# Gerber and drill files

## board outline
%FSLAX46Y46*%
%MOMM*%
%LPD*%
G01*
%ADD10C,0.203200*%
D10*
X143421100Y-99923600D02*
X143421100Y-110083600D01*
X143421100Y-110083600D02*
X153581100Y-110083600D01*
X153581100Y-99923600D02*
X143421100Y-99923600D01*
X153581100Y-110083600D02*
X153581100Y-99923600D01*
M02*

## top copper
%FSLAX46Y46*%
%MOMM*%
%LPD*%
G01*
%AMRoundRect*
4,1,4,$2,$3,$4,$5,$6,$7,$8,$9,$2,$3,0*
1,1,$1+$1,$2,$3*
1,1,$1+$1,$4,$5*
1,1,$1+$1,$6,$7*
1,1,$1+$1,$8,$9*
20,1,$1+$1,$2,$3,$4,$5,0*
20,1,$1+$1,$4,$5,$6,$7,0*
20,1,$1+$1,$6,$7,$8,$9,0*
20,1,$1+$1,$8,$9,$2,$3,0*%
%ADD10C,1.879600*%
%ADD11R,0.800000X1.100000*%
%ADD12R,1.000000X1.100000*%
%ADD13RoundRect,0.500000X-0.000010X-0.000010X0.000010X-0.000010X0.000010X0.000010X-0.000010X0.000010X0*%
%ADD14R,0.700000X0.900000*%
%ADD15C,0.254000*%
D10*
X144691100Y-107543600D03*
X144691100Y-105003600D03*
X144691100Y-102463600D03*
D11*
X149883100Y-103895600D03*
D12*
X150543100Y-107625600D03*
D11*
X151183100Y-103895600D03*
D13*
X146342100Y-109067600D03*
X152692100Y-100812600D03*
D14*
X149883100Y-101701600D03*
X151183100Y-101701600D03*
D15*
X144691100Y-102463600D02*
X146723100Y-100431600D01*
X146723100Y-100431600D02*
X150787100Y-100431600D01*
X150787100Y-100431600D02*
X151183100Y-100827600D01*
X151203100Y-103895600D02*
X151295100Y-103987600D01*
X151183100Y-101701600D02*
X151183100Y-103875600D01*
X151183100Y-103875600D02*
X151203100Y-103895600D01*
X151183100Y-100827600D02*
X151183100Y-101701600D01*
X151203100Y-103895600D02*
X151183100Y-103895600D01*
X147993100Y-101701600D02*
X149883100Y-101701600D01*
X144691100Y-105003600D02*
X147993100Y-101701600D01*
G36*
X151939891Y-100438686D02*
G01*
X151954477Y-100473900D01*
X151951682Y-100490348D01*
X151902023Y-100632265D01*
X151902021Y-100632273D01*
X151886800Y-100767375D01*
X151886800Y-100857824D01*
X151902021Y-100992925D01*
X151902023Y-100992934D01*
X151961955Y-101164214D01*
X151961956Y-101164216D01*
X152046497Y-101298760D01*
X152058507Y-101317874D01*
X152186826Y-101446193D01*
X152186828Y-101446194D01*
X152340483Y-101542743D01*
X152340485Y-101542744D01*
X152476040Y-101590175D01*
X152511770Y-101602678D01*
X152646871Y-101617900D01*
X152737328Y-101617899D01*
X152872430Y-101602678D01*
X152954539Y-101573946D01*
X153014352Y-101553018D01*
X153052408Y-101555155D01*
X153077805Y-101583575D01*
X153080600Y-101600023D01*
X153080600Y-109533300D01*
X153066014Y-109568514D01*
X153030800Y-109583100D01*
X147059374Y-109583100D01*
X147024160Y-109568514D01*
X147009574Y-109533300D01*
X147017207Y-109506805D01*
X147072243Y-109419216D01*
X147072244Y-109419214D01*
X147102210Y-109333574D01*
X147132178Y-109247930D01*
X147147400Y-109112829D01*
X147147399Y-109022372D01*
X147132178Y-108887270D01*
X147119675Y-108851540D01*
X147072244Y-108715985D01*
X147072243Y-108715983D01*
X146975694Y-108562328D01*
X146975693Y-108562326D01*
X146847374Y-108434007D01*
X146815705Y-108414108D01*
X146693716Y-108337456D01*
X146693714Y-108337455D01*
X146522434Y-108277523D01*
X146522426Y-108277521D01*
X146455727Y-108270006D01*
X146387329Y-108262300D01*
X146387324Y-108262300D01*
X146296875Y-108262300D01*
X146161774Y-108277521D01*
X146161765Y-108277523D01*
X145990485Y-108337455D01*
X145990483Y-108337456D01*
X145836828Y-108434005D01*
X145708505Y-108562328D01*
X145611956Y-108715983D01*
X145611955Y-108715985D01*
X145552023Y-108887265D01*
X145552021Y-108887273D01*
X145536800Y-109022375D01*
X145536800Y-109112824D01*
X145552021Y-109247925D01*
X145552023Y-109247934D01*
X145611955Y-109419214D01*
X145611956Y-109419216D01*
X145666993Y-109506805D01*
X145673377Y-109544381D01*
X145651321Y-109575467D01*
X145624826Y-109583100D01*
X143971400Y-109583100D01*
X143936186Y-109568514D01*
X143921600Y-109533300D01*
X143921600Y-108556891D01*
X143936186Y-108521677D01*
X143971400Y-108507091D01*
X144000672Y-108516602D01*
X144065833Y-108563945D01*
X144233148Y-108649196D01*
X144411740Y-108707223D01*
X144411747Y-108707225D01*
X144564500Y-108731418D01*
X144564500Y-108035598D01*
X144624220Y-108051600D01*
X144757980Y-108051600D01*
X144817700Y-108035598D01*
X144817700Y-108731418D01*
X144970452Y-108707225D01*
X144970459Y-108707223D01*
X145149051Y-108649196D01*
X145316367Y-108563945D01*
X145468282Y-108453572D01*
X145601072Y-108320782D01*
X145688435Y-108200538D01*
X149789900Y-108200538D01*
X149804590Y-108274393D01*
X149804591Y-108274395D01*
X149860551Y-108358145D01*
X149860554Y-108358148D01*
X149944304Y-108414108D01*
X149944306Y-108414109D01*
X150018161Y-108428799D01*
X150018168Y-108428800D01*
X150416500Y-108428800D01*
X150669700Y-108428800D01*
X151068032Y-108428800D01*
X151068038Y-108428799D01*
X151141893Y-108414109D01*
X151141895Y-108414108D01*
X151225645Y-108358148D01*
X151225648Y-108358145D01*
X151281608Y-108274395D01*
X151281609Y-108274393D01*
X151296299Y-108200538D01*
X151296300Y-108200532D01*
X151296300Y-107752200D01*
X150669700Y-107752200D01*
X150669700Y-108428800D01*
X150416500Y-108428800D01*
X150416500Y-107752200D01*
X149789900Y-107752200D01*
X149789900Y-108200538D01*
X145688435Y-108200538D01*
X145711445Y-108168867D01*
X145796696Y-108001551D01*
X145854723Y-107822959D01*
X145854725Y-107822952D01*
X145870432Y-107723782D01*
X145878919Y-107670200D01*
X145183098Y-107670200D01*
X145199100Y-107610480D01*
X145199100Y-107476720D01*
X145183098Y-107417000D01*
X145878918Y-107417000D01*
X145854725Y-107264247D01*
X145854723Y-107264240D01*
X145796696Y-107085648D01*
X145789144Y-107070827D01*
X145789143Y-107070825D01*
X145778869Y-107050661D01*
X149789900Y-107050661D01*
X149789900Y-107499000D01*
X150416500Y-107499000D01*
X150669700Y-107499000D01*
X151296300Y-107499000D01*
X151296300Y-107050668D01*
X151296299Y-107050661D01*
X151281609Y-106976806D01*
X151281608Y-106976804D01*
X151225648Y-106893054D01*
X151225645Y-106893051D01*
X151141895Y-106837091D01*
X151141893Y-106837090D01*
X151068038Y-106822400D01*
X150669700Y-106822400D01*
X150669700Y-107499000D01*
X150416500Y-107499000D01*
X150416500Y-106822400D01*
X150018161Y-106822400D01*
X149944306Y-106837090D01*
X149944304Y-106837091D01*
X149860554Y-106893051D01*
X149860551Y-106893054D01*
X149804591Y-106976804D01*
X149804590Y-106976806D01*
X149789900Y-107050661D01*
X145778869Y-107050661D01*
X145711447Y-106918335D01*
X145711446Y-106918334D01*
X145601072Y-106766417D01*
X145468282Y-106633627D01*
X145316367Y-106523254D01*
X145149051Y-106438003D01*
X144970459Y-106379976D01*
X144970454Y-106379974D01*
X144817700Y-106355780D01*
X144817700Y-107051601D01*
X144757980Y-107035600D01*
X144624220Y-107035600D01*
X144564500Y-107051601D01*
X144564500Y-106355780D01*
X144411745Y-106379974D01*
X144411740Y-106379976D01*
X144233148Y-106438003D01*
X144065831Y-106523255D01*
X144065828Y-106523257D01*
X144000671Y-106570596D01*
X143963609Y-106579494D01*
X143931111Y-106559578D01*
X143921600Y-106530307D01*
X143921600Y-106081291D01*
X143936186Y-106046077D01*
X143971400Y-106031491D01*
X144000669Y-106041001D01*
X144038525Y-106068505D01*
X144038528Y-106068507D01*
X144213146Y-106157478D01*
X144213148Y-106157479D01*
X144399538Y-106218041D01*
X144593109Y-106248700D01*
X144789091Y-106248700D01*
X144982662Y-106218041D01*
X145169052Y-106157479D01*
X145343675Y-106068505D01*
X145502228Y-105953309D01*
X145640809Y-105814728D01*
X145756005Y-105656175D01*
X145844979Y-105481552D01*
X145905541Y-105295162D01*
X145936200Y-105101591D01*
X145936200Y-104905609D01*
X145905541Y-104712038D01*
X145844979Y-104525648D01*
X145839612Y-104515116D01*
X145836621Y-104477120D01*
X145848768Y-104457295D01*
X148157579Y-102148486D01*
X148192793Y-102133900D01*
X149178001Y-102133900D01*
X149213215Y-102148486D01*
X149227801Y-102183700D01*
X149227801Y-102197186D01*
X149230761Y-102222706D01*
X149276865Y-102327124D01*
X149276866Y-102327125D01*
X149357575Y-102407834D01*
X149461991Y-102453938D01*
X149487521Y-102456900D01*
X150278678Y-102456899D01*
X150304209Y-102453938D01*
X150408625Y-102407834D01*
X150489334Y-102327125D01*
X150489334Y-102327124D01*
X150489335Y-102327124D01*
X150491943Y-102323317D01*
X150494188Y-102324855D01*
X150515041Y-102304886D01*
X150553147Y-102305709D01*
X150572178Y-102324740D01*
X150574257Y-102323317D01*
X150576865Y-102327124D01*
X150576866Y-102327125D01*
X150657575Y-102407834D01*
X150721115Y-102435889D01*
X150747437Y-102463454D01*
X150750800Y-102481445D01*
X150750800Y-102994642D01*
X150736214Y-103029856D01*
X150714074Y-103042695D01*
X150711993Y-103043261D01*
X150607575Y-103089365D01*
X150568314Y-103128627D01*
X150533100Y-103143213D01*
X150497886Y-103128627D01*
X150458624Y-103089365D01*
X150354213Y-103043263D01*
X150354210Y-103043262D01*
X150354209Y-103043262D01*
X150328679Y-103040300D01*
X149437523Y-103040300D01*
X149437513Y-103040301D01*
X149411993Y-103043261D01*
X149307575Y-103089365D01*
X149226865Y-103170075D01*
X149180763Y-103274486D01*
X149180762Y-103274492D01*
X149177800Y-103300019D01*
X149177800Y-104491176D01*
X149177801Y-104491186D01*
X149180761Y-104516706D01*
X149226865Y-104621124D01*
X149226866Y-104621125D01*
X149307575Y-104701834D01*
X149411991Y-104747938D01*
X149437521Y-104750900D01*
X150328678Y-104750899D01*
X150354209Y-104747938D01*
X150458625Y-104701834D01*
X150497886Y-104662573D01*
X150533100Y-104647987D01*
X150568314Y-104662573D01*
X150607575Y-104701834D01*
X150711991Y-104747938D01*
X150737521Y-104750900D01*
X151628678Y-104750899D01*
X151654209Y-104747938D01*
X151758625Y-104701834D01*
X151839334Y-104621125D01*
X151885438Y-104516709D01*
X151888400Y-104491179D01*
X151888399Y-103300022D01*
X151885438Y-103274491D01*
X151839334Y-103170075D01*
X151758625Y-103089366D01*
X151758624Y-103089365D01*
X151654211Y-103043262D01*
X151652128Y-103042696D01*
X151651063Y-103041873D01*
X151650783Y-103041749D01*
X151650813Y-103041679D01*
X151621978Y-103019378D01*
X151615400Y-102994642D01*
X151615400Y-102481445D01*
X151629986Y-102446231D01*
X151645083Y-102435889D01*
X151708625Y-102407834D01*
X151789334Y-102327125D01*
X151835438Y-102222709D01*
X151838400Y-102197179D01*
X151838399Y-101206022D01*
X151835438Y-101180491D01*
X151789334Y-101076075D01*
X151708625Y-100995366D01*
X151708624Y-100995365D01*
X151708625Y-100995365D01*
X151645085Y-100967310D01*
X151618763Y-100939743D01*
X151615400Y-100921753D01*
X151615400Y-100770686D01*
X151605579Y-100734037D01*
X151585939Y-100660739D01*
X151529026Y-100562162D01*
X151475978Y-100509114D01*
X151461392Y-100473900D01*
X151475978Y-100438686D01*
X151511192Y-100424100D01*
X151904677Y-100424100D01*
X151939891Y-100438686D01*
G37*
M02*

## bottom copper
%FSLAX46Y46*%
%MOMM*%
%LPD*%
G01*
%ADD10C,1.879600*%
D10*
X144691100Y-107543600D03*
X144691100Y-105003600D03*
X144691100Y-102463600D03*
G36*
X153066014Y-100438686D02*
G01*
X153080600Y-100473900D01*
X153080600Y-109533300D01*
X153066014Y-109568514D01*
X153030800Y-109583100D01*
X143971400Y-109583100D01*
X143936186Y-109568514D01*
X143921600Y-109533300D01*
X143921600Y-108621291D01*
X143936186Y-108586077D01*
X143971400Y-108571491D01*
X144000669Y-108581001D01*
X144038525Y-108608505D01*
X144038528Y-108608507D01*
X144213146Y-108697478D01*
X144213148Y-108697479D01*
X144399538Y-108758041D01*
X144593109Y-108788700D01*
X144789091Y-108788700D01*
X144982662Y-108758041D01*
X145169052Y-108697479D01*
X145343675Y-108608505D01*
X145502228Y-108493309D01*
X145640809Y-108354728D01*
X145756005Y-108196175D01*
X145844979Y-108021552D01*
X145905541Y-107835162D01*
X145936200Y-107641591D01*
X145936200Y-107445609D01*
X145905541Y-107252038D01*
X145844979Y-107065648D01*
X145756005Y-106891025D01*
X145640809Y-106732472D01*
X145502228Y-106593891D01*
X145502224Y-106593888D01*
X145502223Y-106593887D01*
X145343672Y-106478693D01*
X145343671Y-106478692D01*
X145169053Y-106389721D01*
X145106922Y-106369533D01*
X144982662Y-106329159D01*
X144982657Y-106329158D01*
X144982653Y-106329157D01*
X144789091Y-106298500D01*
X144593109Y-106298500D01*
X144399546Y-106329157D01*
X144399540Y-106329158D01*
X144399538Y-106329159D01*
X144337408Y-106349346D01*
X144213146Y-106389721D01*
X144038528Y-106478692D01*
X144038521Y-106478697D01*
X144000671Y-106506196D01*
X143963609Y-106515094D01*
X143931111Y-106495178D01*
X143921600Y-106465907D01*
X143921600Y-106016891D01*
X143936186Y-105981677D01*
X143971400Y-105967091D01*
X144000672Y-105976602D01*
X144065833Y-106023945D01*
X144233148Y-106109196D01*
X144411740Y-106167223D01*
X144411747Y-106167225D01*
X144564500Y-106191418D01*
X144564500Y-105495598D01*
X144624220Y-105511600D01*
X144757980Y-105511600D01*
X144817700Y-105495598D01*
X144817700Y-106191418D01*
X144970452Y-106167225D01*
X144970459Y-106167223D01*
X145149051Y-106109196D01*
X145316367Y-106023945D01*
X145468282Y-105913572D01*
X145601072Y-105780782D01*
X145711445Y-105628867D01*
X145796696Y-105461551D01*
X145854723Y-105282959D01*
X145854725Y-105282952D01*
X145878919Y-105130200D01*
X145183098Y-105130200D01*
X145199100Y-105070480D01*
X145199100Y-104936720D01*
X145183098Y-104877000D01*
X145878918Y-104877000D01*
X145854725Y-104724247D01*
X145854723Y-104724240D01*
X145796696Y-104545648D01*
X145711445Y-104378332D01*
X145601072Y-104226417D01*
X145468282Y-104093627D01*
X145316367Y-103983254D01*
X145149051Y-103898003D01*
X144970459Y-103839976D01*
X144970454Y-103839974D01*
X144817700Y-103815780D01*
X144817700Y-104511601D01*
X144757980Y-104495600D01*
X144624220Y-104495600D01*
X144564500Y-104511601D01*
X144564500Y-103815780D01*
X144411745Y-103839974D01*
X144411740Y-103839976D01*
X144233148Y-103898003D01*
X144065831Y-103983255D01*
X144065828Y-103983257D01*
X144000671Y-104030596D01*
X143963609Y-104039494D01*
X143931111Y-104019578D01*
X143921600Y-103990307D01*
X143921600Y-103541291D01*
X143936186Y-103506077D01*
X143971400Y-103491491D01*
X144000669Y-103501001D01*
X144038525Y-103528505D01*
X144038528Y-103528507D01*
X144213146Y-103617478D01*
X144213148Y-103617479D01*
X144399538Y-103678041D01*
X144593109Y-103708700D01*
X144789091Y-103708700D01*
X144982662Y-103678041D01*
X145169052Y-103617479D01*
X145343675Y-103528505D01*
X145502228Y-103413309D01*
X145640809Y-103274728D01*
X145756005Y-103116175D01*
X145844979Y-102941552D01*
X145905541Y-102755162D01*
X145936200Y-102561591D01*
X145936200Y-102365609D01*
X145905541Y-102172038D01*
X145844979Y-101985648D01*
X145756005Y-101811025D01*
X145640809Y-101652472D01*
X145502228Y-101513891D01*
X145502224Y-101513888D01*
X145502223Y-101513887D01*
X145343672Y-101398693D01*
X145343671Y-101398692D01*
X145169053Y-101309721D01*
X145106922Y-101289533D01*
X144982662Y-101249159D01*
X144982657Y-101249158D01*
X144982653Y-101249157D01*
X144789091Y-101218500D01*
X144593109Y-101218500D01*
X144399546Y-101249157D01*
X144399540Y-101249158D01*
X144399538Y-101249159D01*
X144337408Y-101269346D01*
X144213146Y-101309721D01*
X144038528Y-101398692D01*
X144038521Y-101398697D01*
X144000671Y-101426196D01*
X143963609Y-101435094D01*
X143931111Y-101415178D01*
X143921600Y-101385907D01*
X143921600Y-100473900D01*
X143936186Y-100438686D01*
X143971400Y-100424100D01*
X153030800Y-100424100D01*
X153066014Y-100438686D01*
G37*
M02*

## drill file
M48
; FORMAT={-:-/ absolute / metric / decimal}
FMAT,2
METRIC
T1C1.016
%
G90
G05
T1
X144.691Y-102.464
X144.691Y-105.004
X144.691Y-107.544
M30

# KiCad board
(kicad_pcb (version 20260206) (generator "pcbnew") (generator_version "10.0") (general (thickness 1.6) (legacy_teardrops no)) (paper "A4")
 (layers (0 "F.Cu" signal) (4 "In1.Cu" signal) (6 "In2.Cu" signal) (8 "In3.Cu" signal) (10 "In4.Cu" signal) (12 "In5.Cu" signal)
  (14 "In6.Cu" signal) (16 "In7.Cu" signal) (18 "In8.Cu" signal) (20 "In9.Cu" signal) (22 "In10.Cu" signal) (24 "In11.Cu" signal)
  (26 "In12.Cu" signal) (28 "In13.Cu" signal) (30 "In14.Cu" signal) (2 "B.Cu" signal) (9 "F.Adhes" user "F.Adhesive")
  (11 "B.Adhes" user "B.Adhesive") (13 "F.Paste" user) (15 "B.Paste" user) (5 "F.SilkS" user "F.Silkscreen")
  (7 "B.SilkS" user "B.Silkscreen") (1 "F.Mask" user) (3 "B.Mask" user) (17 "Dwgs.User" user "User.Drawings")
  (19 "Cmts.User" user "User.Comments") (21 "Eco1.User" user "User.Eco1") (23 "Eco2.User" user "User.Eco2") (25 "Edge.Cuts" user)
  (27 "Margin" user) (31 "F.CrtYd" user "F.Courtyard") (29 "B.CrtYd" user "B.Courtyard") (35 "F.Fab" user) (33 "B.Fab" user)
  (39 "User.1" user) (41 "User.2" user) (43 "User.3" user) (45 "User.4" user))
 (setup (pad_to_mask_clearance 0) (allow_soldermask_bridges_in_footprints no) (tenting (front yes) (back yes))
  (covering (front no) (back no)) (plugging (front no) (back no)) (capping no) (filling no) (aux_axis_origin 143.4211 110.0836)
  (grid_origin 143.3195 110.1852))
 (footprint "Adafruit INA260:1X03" (layer "F.Cu") (at 144.6911 107.5436 90)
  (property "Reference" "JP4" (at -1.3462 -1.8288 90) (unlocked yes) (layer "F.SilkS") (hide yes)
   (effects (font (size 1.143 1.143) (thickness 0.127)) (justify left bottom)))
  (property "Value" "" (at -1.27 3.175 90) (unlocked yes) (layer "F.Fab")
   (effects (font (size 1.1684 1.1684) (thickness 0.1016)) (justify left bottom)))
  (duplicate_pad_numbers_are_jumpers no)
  (pad "1" thru_hole circle (at 0 0 180) (size 1.8796 1.8796) (drill 1.016) (layers "*.Cu" "*.Mask") (remove_unused_layers no) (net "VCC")
   (solder_mask_margin 0.1016) (thermal_bridge_angle 0))
  (pad "2" thru_hole circle (at 2.54 0 180) (size 1.8796 1.8796) (drill 1.016) (layers "*.Cu" "*.Mask") (remove_unused_layers no)
   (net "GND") (solder_mask_margin 0.1016) (thermal_bridge_angle 0))
  (pad "3" thru_hole circle (at 5.08 0 180) (size 1.8796 1.8796) (drill 1.016) (layers "*.Cu" "*.Mask") (remove_unused_layers no) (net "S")
   (solder_mask_margin 0.1016) (thermal_bridge_angle 0)))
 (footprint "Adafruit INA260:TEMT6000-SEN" (layer "F.Cu") (at 150.5331 105.7656 -90)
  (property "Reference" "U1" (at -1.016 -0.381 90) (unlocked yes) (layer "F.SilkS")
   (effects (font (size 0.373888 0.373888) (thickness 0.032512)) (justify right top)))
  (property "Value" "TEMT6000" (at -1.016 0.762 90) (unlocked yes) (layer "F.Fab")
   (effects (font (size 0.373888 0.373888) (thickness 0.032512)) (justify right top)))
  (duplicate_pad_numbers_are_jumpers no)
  (pad "BASE" smd rect (at -1.87 0.65 270) (size 1.1 0.8) (layers "F.Cu" "F.Mask" "F.Paste") (solder_mask_margin 0.1016)
   (solder_paste_margin 0) (thermal_bridge_angle 0))
  (pad "COLLECTOR" smd rect (at 1.86 -0.01 270) (size 1.1 1) (layers "F.Cu" "F.Mask" "F.Paste") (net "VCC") (solder_mask_margin 0.1016)
   (solder_paste_margin 0) (thermal_bridge_angle 0))
  (pad "EMITTER" smd rect (at -1.87 -0.65 270) (size 1.1 0.8) (layers "F.Cu" "F.Mask" "F.Paste") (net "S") (solder_mask_margin 0.1016)
   (solder_paste_margin 0) (thermal_bridge_angle 0)))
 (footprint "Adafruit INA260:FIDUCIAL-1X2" (layer "F.Cu") (at 146.3421 109.0676)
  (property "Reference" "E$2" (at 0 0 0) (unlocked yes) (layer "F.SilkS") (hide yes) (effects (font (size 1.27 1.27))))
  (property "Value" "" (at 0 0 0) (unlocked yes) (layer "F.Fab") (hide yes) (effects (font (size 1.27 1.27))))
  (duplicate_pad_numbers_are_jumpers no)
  (pad "1" smd roundrect (at 0 0) (size 1 1) (layers "F.Cu" "F.Mask") (roundrect_rratio 0.5) (solder_mask_margin 0.1016)
   (solder_paste_margin 0) (thermal_bridge_angle 0)))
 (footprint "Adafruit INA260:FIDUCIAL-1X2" (layer "F.Cu") (at 152.6921 100.8126)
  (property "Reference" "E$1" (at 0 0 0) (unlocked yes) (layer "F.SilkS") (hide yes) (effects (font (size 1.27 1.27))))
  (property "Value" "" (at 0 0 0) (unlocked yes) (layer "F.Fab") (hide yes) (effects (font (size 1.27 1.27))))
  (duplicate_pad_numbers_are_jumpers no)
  (pad "1" smd roundrect (at 0 0) (size 1 1) (layers "F.Cu" "F.Mask") (roundrect_rratio 0.5) (solder_mask_margin 0.1016)
   (solder_paste_margin 0) (thermal_bridge_angle 0)))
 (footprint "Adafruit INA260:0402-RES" (layer "F.Cu") (at 150.5331 101.7016)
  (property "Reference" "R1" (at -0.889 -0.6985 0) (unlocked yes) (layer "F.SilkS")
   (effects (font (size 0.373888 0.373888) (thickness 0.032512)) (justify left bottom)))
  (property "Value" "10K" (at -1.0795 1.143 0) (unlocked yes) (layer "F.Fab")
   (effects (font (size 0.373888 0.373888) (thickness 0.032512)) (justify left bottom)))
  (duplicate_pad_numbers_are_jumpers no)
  (pad "1" smd rect (at -0.65 0) (size 0.7 0.9) (layers "F.Cu" "F.Mask" "F.Paste") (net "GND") (solder_mask_margin 0.1016)
   (solder_paste_margin 0) (thermal_bridge_angle 0))
  (pad "2" smd rect (at 0.65 0) (size 0.7 0.9) (layers "F.Cu" "F.Mask" "F.Paste") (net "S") (solder_mask_margin 0.1016)
   (solder_paste_margin 0) (thermal_bridge_angle 0)))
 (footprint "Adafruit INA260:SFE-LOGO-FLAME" (layer "B.Cu") (at 149.5171 106.5276 180)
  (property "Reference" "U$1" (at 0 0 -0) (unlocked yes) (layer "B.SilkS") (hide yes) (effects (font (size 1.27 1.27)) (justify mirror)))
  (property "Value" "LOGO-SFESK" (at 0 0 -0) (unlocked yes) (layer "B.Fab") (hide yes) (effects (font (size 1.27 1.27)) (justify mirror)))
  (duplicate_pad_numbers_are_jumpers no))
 (gr_line (start 143.4211 99.9236) (end 143.4211 110.0836) (stroke (width 0.2032) (type solid)) (layer "Edge.Cuts"))
 (gr_line (start 143.4211 110.0836) (end 153.5811 110.0836) (stroke (width 0.2032) (type solid)) (layer "Edge.Cuts"))
 (gr_line (start 153.5811 99.9236) (end 143.4211 99.9236) (stroke (width 0.2032) (type solid)) (layer "Edge.Cuts"))
 (gr_line (start 153.5811 110.0836) (end 153.5811 99.9236) (stroke (width 0.2032) (type solid)) (layer "Edge.Cuts"))
 (segment (start 144.6911 102.4636) (end 146.7231 100.4316) (width 0.254) (layer "F.Cu") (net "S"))
 (segment (start 146.7231 100.4316) (end 150.7871 100.4316) (width 0.254) (layer "F.Cu") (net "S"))
 (segment (start 150.7871 100.4316) (end 151.1831 100.8276) (width 0.254) (layer "F.Cu") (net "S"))
 (segment (start 151.2031 103.8956) (end 151.2951 103.9876) (width 0.254) (layer "F.Cu") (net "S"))
 (segment (start 151.1831 101.7016) (end 151.1831 103.8756) (width 0.254) (layer "F.Cu") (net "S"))
 (segment (start 151.1831 103.8756) (end 151.2031 103.8956) (width 0.254) (layer "F.Cu") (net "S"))
 (segment (start 151.1831 100.8276) (end 151.1831 101.7016) (width 0.254) (layer "F.Cu") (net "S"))
 (segment (start 151.2031 103.8956) (end 151.1831 103.8956) (width 0.254) (layer "F.Cu") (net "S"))
 (segment (start 147.9931 101.7016) (end 149.8831 101.7016) (width 0.254) (layer "F.Cu") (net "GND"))
 (segment (start 144.6911 105.0036) (end 147.9931 101.7016) (width 0.254) (layer "F.Cu") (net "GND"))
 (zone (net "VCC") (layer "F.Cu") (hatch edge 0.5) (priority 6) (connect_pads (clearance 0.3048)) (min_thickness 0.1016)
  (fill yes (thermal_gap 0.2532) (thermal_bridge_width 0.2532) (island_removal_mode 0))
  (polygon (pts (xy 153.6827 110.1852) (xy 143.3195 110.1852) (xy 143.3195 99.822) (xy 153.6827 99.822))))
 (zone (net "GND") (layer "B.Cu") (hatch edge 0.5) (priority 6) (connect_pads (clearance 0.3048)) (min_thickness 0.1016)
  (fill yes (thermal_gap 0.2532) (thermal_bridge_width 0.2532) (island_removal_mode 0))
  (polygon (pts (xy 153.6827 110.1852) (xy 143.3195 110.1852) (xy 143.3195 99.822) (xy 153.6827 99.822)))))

